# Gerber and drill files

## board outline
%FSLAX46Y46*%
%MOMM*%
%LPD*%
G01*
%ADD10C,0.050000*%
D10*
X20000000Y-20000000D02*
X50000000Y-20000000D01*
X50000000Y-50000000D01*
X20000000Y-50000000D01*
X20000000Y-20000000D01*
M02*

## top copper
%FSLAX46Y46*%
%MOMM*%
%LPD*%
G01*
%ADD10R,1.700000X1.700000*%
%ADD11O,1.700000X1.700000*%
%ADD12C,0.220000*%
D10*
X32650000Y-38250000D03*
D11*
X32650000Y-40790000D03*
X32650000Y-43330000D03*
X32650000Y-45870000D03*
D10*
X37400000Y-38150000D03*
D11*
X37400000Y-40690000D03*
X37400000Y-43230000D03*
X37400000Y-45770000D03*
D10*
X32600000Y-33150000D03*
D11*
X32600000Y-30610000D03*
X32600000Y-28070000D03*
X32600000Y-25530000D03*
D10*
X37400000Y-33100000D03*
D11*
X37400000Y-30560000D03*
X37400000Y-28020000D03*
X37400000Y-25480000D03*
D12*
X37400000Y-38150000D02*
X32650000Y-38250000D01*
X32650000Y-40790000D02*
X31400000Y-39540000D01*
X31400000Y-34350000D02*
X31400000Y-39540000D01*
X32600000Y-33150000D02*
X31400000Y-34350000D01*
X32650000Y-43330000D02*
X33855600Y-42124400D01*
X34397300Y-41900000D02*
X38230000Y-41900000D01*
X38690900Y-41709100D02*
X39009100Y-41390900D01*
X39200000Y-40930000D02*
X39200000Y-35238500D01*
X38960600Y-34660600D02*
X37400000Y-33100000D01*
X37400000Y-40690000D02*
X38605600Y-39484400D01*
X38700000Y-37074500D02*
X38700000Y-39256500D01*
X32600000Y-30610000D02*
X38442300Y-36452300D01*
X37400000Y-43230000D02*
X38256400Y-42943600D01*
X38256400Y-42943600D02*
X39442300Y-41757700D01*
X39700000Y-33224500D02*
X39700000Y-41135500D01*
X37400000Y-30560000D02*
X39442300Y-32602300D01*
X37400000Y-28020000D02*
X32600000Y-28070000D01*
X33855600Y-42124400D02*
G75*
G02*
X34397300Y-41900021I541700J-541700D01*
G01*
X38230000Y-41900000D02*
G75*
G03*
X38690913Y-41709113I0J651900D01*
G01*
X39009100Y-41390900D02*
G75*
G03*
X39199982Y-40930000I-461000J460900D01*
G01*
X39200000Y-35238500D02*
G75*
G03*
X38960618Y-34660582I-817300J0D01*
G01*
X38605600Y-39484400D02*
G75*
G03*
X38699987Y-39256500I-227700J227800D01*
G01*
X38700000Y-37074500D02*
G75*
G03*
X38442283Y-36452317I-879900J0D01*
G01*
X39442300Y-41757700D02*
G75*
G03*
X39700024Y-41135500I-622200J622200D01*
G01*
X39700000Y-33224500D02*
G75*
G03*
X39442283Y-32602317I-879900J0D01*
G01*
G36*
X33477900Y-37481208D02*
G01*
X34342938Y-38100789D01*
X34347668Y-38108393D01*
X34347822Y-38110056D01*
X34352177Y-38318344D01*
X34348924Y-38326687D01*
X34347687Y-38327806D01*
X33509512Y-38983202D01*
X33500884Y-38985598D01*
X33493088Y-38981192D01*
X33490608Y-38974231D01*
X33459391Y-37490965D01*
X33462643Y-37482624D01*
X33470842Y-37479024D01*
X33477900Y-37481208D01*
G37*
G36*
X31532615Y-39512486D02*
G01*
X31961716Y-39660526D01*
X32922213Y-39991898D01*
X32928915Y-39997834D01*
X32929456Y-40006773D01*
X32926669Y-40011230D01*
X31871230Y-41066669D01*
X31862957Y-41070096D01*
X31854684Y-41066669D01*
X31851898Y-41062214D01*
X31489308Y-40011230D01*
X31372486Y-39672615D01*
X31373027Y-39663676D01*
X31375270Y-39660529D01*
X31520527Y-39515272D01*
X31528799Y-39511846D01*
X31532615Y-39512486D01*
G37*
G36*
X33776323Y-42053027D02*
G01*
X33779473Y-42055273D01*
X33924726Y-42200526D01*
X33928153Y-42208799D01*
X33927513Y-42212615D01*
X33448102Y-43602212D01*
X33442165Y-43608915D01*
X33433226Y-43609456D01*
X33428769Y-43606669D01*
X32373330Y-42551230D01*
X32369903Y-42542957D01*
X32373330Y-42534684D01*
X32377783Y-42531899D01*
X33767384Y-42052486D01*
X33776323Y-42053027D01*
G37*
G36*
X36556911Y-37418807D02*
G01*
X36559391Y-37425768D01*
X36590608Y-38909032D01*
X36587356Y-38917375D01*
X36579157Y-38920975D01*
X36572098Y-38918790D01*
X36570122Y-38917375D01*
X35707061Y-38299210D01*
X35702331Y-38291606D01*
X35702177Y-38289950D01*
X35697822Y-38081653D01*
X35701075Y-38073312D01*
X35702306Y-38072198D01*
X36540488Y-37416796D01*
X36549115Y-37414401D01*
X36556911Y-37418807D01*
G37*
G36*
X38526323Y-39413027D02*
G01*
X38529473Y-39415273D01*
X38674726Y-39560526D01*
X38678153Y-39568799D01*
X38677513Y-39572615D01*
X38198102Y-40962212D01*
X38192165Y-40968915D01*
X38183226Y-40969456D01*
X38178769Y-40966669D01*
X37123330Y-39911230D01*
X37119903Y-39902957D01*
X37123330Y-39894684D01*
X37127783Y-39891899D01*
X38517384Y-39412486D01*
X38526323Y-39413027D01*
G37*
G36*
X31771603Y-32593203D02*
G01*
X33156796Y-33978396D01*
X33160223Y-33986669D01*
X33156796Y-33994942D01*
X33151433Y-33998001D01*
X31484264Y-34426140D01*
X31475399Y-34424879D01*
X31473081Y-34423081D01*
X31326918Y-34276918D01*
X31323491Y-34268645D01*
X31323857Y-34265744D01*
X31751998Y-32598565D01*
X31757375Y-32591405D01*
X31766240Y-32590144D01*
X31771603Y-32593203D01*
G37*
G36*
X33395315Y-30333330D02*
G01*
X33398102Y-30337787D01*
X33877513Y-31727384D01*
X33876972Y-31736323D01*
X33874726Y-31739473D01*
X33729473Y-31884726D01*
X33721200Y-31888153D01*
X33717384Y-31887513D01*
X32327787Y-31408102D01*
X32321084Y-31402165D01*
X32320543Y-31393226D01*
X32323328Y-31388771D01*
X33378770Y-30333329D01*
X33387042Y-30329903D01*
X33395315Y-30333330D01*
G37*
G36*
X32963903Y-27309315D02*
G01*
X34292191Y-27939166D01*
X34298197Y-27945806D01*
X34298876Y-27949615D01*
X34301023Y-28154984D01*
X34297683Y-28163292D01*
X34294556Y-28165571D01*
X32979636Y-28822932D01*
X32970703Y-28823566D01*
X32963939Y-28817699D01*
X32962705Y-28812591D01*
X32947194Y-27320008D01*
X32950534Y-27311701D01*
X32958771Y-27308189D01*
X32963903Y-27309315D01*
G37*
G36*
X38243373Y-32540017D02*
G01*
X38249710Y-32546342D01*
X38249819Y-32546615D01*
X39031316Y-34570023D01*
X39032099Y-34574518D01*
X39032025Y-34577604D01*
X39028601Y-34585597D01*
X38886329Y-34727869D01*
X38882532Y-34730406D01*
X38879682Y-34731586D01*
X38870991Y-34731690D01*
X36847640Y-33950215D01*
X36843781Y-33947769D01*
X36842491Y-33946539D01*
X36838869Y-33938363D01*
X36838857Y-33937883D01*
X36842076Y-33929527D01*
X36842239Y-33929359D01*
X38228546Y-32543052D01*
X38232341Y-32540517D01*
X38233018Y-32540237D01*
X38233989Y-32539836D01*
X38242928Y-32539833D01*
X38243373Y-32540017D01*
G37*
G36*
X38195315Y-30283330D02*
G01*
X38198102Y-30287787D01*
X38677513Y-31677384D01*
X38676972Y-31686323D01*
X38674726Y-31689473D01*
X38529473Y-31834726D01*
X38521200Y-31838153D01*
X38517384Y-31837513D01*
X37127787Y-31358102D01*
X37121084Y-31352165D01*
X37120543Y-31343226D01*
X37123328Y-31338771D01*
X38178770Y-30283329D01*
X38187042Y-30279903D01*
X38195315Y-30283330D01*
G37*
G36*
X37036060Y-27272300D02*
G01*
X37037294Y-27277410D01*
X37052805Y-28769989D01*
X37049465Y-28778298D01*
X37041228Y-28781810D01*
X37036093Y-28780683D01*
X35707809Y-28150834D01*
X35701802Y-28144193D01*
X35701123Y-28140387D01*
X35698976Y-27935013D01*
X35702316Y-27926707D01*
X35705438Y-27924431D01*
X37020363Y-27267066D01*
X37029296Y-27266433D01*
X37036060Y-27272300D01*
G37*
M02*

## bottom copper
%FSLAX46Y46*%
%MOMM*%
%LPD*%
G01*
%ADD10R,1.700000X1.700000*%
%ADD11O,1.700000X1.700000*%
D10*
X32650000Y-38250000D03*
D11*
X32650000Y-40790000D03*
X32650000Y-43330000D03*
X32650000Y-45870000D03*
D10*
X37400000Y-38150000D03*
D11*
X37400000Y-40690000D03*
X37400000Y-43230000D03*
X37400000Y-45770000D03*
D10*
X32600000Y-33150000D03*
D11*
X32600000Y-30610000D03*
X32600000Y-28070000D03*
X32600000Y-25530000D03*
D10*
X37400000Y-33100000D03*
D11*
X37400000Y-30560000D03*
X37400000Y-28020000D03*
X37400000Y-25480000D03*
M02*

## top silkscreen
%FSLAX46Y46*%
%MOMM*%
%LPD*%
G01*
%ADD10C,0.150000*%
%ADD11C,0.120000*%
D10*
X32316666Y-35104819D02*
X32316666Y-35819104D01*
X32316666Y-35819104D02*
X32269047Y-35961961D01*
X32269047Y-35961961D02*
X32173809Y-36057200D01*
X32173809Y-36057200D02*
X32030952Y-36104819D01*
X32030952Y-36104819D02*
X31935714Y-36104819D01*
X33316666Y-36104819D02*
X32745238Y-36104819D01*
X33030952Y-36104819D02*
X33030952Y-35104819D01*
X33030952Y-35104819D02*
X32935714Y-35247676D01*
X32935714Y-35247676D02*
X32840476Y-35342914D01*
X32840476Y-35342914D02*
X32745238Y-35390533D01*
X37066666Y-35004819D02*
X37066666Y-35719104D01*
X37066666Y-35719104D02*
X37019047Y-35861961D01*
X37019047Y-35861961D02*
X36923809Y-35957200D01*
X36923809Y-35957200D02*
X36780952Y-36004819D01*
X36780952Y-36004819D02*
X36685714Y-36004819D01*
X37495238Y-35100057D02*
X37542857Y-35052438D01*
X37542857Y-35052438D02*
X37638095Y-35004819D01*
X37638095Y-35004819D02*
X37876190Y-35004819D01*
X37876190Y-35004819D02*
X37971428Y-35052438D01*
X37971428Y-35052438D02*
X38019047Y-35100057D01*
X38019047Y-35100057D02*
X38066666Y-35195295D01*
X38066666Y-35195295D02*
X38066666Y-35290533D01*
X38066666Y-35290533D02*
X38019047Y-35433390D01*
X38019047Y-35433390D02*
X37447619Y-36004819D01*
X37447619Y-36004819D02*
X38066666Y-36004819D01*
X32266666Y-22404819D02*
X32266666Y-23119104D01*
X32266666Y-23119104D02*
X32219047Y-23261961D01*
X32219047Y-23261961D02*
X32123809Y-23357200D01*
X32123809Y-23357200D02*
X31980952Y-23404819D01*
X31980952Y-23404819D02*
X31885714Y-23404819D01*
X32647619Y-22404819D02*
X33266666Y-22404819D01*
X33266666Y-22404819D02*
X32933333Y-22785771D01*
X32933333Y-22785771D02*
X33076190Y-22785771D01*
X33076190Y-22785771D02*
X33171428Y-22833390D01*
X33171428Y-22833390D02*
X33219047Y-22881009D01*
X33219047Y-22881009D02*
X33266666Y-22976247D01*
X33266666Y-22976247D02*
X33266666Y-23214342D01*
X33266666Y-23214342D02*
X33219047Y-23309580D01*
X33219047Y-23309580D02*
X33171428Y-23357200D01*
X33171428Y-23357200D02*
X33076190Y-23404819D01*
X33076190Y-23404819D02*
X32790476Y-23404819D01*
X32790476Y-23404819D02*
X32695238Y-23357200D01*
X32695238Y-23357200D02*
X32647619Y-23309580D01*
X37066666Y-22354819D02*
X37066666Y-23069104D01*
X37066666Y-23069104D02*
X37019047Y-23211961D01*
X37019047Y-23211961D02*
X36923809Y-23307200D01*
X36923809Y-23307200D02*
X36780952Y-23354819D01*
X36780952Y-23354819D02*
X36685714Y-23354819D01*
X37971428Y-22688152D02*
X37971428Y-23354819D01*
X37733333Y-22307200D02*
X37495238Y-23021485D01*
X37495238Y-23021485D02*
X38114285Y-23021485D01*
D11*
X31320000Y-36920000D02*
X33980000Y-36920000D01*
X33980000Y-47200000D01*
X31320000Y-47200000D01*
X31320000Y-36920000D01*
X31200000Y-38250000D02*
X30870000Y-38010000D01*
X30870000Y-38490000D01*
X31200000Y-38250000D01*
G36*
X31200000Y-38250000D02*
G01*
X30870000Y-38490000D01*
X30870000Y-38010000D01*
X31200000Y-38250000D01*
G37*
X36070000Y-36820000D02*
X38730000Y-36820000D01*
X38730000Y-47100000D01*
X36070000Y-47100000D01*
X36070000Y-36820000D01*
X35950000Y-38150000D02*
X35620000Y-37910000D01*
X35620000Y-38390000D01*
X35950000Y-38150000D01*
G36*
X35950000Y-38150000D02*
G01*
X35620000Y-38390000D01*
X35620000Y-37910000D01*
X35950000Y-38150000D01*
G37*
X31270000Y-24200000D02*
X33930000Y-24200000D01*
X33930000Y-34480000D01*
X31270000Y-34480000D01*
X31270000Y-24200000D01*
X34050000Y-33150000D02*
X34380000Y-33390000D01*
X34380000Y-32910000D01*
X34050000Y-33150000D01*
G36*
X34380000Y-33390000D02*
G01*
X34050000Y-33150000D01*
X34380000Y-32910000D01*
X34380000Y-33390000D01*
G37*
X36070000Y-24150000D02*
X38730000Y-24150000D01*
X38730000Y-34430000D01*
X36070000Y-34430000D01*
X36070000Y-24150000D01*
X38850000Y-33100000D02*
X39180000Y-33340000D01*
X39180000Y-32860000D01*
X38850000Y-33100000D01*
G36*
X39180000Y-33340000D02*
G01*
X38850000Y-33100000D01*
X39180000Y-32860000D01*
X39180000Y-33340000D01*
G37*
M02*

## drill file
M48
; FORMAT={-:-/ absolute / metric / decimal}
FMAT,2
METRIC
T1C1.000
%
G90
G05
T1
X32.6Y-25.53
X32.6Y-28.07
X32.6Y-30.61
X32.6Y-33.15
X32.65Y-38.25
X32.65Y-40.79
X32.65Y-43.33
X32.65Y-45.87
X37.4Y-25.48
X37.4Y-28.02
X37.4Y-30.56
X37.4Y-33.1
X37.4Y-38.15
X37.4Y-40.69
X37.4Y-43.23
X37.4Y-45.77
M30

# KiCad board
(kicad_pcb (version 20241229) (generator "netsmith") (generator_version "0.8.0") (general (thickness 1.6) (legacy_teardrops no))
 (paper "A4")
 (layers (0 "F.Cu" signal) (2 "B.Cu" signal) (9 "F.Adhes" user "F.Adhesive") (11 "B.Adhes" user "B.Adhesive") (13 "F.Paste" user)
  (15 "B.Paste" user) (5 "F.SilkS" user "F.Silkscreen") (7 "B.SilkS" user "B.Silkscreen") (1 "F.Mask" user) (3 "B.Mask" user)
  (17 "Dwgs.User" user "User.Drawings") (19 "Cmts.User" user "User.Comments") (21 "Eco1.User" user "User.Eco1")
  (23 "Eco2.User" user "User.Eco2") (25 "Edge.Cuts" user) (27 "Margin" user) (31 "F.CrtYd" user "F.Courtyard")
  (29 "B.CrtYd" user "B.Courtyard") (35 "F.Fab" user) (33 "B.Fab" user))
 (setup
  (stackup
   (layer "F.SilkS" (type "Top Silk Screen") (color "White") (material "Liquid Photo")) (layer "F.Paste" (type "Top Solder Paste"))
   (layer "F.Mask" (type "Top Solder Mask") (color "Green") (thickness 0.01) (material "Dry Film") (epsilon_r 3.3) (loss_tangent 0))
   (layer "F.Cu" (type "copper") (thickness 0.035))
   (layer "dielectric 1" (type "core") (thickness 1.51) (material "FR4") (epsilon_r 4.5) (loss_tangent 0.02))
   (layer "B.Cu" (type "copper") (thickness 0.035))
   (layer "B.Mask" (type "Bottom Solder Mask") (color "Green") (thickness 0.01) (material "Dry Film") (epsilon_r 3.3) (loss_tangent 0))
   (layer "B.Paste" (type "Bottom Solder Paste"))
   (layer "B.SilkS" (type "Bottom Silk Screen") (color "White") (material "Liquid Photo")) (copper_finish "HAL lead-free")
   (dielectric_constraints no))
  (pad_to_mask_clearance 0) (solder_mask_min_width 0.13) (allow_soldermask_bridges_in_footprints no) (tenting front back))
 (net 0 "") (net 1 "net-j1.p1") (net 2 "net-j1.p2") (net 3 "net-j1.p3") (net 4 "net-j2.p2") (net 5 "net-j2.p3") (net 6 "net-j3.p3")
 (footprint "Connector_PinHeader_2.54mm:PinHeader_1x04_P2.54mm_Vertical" (layer "F.Cu") (at 32.65 38.25)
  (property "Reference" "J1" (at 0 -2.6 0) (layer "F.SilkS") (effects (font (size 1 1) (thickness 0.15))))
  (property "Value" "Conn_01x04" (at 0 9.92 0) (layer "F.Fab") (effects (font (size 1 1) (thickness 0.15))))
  (pad "1" thru_hole rect (at 0 0) (size 1.7 1.7) (drill 1) (layers "*.Cu" "*.Mask") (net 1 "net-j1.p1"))
  (pad "2" thru_hole oval (at 0 2.54) (size 1.7 1.7) (drill 1) (layers "*.Cu" "*.Mask") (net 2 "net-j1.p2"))
  (pad "3" thru_hole oval (at 0 5.08) (size 1.7 1.7) (drill 1) (layers "*.Cu" "*.Mask") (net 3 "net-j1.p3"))
  (pad "4" thru_hole oval (at 0 7.62) (size 1.7 1.7) (drill 1) (layers "*.Cu" "*.Mask"))
  (fp_rect (start -1.33 -1.33) (end 1.33 8.95) (stroke (width 0.12) (type solid)) (fill no) (layer "F.SilkS"))
  (fp_poly (pts (xy -1.45 0) (xy -1.78 -0.24) (xy -1.78 0.24)) (stroke (width 0.12) (type solid)) (fill solid) (layer "F.SilkS")))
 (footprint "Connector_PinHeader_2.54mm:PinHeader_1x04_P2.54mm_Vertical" (layer "F.Cu") (at 37.4 38.15)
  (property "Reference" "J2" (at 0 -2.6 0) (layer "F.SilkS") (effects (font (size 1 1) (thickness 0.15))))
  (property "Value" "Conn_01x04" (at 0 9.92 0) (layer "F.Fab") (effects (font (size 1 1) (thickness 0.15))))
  (pad "1" thru_hole rect (at 0 0) (size 1.7 1.7) (drill 1) (layers "*.Cu" "*.Mask") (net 1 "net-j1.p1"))
  (pad "2" thru_hole oval (at 0 2.54) (size 1.7 1.7) (drill 1) (layers "*.Cu" "*.Mask") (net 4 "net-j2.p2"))
  (pad "3" thru_hole oval (at 0 5.08) (size 1.7 1.7) (drill 1) (layers "*.Cu" "*.Mask") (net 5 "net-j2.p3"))
  (pad "4" thru_hole oval (at 0 7.62) (size 1.7 1.7) (drill 1) (layers "*.Cu" "*.Mask"))
  (fp_rect (start -1.33 -1.33) (end 1.33 8.95) (stroke (width 0.12) (type solid)) (fill no) (layer "F.SilkS"))
  (fp_poly (pts (xy -1.45 0) (xy -1.78 -0.24) (xy -1.78 0.24)) (stroke (width 0.12) (type solid)) (fill solid) (layer "F.SilkS")))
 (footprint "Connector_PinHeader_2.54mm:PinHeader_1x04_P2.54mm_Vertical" (layer "F.Cu") (at 32.6 33.15 180)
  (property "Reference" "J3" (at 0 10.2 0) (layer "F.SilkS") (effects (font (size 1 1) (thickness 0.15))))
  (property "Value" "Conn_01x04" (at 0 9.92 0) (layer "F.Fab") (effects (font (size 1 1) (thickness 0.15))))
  (pad "1" thru_hole rect (at 0 0 180) (size 1.7 1.7) (drill 1) (layers "*.Cu" "*.Mask") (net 2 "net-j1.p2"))
  (pad "2" thru_hole oval (at 0 2.54 180) (size 1.7 1.7) (drill 1) (layers "*.Cu" "*.Mask") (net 4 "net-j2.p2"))
  (pad "3" thru_hole oval (at 0 5.08 180) (size 1.7 1.7) (drill 1) (layers "*.Cu" "*.Mask") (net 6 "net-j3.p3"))
  (pad "4" thru_hole oval (at 0 7.62 180) (size 1.7 1.7) (drill 1) (layers "*.Cu" "*.Mask"))
  (fp_rect (start -1.33 -1.33) (end 1.33 8.95) (stroke (width 0.12) (type solid)) (fill no) (layer "F.SilkS"))
  (fp_poly (pts (xy -1.45 0) (xy -1.78 -0.24) (xy -1.78 0.24)) (stroke (width 0.12) (type solid)) (fill solid) (layer "F.SilkS")))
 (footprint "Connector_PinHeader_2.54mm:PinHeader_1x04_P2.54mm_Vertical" (layer "F.Cu") (at 37.4 33.1 180)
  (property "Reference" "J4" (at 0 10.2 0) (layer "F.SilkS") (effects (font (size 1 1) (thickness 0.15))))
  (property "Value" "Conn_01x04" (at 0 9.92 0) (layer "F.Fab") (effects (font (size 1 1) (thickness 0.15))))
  (pad "1" thru_hole rect (at 0 0 180) (size 1.7 1.7) (drill 1) (layers "*.Cu" "*.Mask") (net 3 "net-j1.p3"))
  (pad "2" thru_hole oval (at 0 2.54 180) (size 1.7 1.7) (drill 1) (layers "*.Cu" "*.Mask") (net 5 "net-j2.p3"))
  (pad "3" thru_hole oval (at 0 5.08 180) (size 1.7 1.7) (drill 1) (layers "*.Cu" "*.Mask") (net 6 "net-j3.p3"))
  (pad "4" thru_hole oval (at 0 7.62 180) (size 1.7 1.7) (drill 1) (layers "*.Cu" "*.Mask"))
  (fp_rect (start -1.33 -1.33) (end 1.33 8.95) (stroke (width 0.12) (type solid)) (fill no) (layer "F.SilkS"))
  (fp_poly (pts (xy -1.45 0) (xy -1.78 -0.24) (xy -1.78 0.24)) (stroke (width 0.12) (type solid)) (fill solid) (layer "F.SilkS")))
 (segment (start 37.4 38.15) (end 32.65 38.25) (width 0.22) (layer "F.Cu") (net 1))
 (segment (start 32.65 40.79) (end 31.4 39.54) (width 0.22) (layer "F.Cu") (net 2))
 (segment (start 31.4 34.35) (end 31.4 39.54) (width 0.22) (layer "F.Cu") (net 2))
 (segment (start 32.6 33.15) (end 31.4 34.35) (width 0.22) (layer "F.Cu") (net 2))
 (segment (start 32.65 43.33) (end 33.8556 42.1244) (width 0.22) (layer "F.Cu") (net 3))
 (segment (start 34.3973 41.9) (end 38.23 41.9) (width 0.22) (layer "F.Cu") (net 3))
 (segment (start 38.6909 41.7091) (end 39.0091 41.3909) (width 0.22) (layer "F.Cu") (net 3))
 (segment (start 39.2 40.93) (end 39.2 35.2385) (width 0.22) (layer "F.Cu") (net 3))
 (segment (start 38.9606 34.6606) (end 37.4 33.1) (width 0.22) (layer "F.Cu") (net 3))
 (segment (start 37.4 40.69) (end 38.6056 39.4844) (width 0.22) (layer "F.Cu") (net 4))
 (segment (start 38.7 37.0745) (end 38.7 39.2565) (width 0.22) (layer "F.Cu") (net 4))
 (segment (start 32.6 30.61) (end 38.4423 36.4523) (width 0.22) (layer "F.Cu") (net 4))
 (segment (start 37.4 43.23) (end 38.2564 42.9436) (width 0.22) (layer "F.Cu") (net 5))
 (segment (start 38.2564 42.9436) (end 39.4423 41.7577) (width 0.22) (layer "F.Cu") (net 5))
 (segment (start 39.7 33.2245) (end 39.7 41.1355) (width 0.22) (layer "F.Cu") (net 5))
 (segment (start 37.4 30.56) (end 39.4423 32.6023) (width 0.22) (layer "F.Cu") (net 5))
 (segment (start 37.4 28.02) (end 32.6 28.07) (width 0.22) (layer "F.Cu") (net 6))
 (arc (start 33.8556 42.1244) (mid 34.1042 41.9583) (end 34.3973 41.9) (width 0.22) (layer "F.Cu") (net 3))
 (arc (start 38.23 41.9) (mid 38.4794 41.8504) (end 38.6909 41.7091) (width 0.22) (layer "F.Cu") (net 3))
 (arc (start 39.0091 41.3909) (mid 39.1504 41.1794) (end 39.2 40.93) (width 0.22) (layer "F.Cu") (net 3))
 (arc (start 39.2 35.2385) (mid 39.1378 34.9258) (end 38.9606 34.6606) (width 0.22) (layer "F.Cu") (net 3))
 (arc (start 38.6056 39.4844) (mid 38.6755 39.3798) (end 38.7 39.2565) (width 0.22) (layer "F.Cu") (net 4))
 (arc (start 38.7 37.0745) (mid 38.633 36.7377) (end 38.4423 36.4523) (width 0.22) (layer "F.Cu") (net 4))
 (arc (start 39.4423 41.7577) (mid 39.633 41.4723) (end 39.7 41.1355) (width 0.22) (layer "F.Cu") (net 5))
 (arc (start 39.7 33.2245) (mid 39.633 32.8877) (end 39.4423 32.6023) (width 0.22) (layer "F.Cu") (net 5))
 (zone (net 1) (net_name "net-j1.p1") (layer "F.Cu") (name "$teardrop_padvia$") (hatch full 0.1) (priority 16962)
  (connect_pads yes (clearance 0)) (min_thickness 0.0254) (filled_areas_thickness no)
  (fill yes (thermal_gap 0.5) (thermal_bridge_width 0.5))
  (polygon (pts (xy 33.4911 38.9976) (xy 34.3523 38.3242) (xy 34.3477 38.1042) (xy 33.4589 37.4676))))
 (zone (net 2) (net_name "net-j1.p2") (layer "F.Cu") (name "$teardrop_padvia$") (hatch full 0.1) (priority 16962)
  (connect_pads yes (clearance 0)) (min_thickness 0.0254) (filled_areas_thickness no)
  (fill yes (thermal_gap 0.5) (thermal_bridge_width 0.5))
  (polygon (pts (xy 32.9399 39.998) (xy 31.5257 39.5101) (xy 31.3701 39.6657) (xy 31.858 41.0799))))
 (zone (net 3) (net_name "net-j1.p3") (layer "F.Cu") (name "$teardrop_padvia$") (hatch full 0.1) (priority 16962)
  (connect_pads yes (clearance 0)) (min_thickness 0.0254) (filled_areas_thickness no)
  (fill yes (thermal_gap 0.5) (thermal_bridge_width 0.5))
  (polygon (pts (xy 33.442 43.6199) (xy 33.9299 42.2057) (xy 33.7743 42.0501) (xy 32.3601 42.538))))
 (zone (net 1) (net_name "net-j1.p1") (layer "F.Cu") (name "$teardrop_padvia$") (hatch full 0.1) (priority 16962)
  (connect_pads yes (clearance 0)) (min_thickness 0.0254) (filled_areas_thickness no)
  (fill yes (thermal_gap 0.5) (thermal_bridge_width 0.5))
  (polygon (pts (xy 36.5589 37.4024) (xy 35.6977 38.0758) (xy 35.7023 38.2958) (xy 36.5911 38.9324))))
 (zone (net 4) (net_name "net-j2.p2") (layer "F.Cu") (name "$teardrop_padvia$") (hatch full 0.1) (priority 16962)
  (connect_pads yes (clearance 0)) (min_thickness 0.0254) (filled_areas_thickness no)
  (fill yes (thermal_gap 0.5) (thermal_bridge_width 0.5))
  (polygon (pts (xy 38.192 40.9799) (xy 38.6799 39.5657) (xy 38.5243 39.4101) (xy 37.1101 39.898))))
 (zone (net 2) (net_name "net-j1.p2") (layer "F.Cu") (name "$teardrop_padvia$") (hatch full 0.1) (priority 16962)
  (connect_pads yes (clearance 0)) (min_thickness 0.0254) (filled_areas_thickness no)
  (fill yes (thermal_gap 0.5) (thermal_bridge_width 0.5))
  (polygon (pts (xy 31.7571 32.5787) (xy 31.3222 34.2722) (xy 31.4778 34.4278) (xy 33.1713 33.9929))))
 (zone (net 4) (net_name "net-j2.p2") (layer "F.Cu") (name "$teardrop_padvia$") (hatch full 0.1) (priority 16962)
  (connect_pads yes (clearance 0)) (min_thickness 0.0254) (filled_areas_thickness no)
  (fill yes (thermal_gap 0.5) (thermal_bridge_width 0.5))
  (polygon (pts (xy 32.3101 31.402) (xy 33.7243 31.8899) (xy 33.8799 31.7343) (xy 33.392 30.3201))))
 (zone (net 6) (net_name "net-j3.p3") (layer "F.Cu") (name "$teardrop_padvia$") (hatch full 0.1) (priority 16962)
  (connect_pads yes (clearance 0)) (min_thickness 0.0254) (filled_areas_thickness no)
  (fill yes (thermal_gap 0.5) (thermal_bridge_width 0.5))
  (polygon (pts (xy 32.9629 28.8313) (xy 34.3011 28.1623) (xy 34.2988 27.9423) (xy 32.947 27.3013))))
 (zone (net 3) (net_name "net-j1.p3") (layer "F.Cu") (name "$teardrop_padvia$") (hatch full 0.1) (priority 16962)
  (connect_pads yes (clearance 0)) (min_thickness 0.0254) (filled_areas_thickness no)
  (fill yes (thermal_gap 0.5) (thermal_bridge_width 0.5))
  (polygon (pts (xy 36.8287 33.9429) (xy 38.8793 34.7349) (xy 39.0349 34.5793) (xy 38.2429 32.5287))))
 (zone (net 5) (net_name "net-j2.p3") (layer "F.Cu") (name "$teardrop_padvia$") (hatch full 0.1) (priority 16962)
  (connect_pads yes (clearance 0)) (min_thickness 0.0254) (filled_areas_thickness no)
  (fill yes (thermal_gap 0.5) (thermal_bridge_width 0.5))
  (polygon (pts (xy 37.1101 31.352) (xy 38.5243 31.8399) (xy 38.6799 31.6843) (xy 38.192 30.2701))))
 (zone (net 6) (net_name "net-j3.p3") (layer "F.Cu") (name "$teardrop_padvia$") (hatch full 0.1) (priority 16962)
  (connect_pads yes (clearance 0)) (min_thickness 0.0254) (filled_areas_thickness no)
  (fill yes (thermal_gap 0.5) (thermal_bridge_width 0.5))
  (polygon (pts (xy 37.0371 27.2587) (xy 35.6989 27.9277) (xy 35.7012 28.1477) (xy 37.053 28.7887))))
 (gr_rect (start 20 20) (end 50 50) (stroke (width 0.05) (type default)) (fill no) (layer "Edge.Cuts")))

